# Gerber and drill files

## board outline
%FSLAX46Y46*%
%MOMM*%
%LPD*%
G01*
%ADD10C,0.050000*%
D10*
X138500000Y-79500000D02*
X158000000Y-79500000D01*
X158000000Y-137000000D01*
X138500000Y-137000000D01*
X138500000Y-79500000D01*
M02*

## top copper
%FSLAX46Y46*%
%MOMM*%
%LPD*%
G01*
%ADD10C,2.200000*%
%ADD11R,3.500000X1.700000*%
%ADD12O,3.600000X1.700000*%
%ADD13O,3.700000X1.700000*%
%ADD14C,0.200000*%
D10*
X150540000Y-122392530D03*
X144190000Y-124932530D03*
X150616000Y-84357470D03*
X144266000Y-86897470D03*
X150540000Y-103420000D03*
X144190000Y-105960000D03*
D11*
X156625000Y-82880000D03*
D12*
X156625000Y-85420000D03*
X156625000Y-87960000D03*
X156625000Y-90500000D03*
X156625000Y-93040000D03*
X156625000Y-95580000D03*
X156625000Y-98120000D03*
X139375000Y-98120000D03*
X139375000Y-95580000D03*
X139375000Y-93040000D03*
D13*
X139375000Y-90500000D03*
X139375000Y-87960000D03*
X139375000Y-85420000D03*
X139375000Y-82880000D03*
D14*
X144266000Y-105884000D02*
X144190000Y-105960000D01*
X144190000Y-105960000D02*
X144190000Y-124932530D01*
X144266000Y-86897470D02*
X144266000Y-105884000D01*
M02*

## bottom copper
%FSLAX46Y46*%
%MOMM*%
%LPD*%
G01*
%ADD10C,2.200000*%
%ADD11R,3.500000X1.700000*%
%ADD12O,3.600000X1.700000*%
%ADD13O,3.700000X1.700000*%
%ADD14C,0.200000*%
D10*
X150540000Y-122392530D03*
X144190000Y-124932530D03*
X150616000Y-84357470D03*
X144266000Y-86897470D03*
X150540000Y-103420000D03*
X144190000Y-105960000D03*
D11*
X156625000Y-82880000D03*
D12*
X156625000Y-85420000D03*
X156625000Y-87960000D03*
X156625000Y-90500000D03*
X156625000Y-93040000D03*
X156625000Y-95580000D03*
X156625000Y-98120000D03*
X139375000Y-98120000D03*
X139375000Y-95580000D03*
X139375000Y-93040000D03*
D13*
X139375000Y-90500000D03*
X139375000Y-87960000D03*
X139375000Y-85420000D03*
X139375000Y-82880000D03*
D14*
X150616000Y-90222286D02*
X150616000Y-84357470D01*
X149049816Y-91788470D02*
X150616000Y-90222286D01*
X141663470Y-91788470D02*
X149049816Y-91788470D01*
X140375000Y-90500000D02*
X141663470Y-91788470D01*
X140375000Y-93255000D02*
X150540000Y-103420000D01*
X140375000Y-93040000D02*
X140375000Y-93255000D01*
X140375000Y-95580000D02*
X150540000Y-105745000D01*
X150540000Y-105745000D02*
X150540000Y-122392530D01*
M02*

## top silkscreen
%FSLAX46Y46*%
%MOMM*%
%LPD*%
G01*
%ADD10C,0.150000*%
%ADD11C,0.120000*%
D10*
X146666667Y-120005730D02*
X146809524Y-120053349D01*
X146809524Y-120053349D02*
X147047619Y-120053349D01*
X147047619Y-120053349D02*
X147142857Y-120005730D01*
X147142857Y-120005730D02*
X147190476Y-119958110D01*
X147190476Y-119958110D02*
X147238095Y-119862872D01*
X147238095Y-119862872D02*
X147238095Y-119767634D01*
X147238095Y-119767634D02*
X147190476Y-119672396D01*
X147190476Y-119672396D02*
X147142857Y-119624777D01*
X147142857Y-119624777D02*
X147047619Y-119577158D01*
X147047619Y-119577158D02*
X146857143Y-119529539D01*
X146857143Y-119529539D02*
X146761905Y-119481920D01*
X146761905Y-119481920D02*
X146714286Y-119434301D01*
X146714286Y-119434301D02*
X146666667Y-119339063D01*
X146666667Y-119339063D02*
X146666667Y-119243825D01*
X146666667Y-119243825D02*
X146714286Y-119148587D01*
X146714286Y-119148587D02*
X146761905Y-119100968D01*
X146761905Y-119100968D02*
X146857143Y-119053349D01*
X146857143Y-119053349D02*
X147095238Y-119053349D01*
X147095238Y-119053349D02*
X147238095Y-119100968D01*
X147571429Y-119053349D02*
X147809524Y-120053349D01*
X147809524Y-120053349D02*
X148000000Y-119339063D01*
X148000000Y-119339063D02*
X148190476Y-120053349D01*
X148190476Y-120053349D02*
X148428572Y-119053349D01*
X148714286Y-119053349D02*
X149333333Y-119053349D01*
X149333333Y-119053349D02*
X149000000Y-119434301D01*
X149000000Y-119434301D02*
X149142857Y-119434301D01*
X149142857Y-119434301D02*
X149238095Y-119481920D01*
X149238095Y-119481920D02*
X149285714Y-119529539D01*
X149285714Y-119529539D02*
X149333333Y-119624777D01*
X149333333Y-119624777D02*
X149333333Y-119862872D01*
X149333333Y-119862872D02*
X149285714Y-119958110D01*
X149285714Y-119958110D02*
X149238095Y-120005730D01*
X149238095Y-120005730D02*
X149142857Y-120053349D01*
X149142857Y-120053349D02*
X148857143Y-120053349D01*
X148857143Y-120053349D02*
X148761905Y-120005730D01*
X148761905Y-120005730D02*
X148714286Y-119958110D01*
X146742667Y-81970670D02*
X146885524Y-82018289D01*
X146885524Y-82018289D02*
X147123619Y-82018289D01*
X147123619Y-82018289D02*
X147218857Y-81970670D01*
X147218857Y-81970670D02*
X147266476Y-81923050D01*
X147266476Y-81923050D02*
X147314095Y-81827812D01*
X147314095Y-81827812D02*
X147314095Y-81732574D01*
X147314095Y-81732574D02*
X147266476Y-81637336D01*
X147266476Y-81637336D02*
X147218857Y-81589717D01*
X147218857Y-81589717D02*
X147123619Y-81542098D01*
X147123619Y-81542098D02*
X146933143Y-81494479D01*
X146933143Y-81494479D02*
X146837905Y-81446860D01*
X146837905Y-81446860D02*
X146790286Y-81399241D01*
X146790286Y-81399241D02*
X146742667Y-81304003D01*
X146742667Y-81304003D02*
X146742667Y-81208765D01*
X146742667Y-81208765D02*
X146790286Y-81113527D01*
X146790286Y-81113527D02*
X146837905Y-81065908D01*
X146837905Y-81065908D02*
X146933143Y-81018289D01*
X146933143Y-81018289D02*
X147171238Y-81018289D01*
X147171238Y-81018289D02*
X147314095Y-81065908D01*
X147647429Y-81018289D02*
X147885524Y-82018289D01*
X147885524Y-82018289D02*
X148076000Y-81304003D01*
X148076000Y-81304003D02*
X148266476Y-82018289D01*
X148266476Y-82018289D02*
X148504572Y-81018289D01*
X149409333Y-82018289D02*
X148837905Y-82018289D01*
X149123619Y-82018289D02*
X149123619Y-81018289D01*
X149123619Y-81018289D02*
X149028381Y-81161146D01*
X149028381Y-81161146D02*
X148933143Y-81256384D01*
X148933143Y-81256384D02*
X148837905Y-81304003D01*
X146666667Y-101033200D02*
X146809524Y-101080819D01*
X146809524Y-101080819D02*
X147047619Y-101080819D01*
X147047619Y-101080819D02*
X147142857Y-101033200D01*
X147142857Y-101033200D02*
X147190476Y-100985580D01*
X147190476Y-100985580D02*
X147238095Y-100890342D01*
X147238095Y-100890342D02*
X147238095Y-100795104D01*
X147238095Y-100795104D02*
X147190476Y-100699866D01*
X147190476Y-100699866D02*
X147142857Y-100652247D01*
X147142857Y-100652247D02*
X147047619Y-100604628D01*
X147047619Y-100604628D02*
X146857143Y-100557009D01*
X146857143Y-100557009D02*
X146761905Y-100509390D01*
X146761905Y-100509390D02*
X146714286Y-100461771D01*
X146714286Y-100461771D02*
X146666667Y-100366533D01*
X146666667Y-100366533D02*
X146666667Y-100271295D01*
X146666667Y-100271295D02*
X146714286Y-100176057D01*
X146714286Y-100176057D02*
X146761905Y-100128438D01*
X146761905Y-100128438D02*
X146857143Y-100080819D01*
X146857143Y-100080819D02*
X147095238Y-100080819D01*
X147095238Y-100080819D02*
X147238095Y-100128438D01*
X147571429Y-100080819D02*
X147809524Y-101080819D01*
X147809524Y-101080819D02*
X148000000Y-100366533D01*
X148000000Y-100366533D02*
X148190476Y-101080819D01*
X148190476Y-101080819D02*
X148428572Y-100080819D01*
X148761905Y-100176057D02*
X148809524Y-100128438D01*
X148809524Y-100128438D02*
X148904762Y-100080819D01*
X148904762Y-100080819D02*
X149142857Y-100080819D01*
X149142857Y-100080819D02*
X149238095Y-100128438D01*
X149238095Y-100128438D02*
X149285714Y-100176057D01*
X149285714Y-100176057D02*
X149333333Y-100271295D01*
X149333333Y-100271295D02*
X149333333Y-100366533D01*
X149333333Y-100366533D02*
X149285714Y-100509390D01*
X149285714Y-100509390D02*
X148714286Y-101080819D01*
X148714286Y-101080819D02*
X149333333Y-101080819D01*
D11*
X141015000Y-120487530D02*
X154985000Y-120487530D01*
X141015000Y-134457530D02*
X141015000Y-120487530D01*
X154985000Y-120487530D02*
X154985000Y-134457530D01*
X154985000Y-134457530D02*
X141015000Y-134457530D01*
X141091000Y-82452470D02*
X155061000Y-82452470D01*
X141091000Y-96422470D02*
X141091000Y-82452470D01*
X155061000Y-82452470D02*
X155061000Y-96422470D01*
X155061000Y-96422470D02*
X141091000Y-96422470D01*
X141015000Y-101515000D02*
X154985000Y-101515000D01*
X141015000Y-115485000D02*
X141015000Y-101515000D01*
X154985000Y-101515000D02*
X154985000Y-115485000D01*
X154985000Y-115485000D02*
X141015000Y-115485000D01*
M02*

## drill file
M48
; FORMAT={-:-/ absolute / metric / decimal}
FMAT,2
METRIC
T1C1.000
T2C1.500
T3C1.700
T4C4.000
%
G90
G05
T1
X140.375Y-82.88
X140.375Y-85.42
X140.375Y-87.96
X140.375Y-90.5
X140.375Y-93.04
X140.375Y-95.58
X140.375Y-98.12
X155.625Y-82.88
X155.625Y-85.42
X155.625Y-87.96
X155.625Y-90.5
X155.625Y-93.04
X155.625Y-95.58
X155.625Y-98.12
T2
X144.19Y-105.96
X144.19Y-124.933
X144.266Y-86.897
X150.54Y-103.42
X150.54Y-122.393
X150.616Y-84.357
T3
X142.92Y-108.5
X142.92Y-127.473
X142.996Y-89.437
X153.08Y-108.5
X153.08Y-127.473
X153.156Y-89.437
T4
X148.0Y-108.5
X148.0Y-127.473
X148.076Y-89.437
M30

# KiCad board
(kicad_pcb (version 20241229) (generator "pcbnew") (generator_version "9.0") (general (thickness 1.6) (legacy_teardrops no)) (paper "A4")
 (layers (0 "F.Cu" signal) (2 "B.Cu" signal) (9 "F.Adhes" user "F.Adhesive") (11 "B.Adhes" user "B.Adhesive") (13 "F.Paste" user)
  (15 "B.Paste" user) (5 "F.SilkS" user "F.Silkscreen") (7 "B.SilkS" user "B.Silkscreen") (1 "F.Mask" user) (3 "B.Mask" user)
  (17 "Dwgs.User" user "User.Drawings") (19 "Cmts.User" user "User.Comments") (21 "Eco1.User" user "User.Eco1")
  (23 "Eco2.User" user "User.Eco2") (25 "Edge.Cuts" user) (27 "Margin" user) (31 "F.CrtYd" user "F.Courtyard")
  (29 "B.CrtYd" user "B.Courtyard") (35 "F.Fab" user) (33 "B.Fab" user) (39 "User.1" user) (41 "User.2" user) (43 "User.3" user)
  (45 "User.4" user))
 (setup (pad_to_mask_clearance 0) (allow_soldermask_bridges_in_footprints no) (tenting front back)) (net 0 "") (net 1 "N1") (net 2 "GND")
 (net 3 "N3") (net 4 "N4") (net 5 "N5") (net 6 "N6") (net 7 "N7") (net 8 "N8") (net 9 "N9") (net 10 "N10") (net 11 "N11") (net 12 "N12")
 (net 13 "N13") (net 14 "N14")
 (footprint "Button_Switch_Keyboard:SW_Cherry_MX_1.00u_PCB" (layer "F.Cu") (at 150.54 122.39253)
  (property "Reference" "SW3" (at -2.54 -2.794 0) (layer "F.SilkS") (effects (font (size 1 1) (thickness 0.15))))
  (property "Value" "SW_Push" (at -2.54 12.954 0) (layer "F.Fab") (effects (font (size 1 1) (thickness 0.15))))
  (fp_line (start -9.525 -1.905) (end 4.445 -1.905) (stroke (width 0.12) (type solid)) (layer "F.SilkS"))
  (fp_line (start -9.525 12.065) (end -9.525 -1.905) (stroke (width 0.12) (type solid)) (layer "F.SilkS"))
  (fp_line (start 4.445 -1.905) (end 4.445 12.065) (stroke (width 0.12) (type solid)) (layer "F.SilkS"))
  (fp_line (start 4.445 12.065) (end -9.525 12.065) (stroke (width 0.12) (type solid)) (layer "F.SilkS"))
  (pad "" np_thru_hole circle (at -7.62 5.08) (size 1.7 1.7) (drill 1.7) (layers "*.Cu" "*.Mask"))
  (pad "" np_thru_hole circle (at -2.54 5.08) (size 4 4) (drill 4) (layers "*.Cu" "*.Mask"))
  (pad "" np_thru_hole circle (at 2.54 5.08) (size 1.7 1.7) (drill 1.7) (layers "*.Cu" "*.Mask"))
  (pad "1" thru_hole circle (at 0 0) (size 2.2 2.2) (drill 1.5) (layers "*.Cu" "*.Mask") (remove_unused_layers no) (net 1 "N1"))
  (pad "2" thru_hole circle (at -6.35 2.54) (size 2.2 2.2) (drill 1.5) (layers "*.Cu" "*.Mask") (remove_unused_layers no) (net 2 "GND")))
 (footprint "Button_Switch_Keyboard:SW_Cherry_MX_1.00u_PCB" (layer "F.Cu") (at 150.616 84.35747)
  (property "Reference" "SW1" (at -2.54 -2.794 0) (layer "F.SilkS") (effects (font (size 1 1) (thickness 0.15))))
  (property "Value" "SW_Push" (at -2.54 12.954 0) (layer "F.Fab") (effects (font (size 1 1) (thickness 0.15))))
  (fp_line (start -9.525 -1.905) (end 4.445 -1.905) (stroke (width 0.12) (type solid)) (layer "F.SilkS"))
  (fp_line (start -9.525 12.065) (end -9.525 -1.905) (stroke (width 0.12) (type solid)) (layer "F.SilkS"))
  (fp_line (start 4.445 -1.905) (end 4.445 12.065) (stroke (width 0.12) (type solid)) (layer "F.SilkS"))
  (fp_line (start 4.445 12.065) (end -9.525 12.065) (stroke (width 0.12) (type solid)) (layer "F.SilkS"))
  (pad "" np_thru_hole circle (at -7.62 5.08) (size 1.7 1.7) (drill 1.7) (layers "*.Cu" "*.Mask"))
  (pad "" np_thru_hole circle (at -2.54 5.08) (size 4 4) (drill 4) (layers "*.Cu" "*.Mask"))
  (pad "" np_thru_hole circle (at 2.54 5.08) (size 1.7 1.7) (drill 1.7) (layers "*.Cu" "*.Mask"))
  (pad "1" thru_hole circle (at 0 0) (size 2.2 2.2) (drill 1.5) (layers "*.Cu" "*.Mask") (remove_unused_layers no) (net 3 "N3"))
  (pad "2" thru_hole circle (at -6.35 2.54) (size 2.2 2.2) (drill 1.5) (layers "*.Cu" "*.Mask") (remove_unused_layers no) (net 2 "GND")))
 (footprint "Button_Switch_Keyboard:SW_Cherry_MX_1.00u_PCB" (layer "F.Cu") (at 150.54 103.42)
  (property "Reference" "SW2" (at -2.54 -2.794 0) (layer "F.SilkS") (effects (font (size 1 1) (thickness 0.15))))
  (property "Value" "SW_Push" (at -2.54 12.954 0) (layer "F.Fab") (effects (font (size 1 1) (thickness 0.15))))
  (fp_line (start -9.525 -1.905) (end 4.445 -1.905) (stroke (width 0.12) (type solid)) (layer "F.SilkS"))
  (fp_line (start -9.525 12.065) (end -9.525 -1.905) (stroke (width 0.12) (type solid)) (layer "F.SilkS"))
  (fp_line (start 4.445 -1.905) (end 4.445 12.065) (stroke (width 0.12) (type solid)) (layer "F.SilkS"))
  (fp_line (start 4.445 12.065) (end -9.525 12.065) (stroke (width 0.12) (type solid)) (layer "F.SilkS"))
  (pad "" np_thru_hole circle (at -7.62 5.08) (size 1.7 1.7) (drill 1.7) (layers "*.Cu" "*.Mask"))
  (pad "" np_thru_hole circle (at -2.54 5.08) (size 4 4) (drill 4) (layers "*.Cu" "*.Mask"))
  (pad "" np_thru_hole circle (at 2.54 5.08) (size 1.7 1.7) (drill 1.7) (layers "*.Cu" "*.Mask"))
  (pad "1" thru_hole circle (at 0 0) (size 2.2 2.2) (drill 1.5) (layers "*.Cu" "*.Mask") (remove_unused_layers no) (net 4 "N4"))
  (pad "2" thru_hole circle (at -6.35 2.54) (size 2.2 2.2) (drill 1.5) (layers "*.Cu" "*.Mask") (remove_unused_layers no) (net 2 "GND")))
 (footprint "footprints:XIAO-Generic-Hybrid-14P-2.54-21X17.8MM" (layer "B.Cu") (at 148 90.5 180)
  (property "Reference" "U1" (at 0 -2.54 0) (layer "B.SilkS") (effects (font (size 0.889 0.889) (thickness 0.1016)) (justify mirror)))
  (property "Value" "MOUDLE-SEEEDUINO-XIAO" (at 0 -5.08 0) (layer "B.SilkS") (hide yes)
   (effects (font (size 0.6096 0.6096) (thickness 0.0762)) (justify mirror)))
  (pad "1" thru_hole rect (at -7.625 7.62 180) (size 3.5 1.7) (drill 1 (offset -1 0)) (layers "*.Cu" "*.Mask") (remove_unused_layers no)
   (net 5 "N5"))
  (pad "2" thru_hole oval (at -7.625 5.08 180) (size 3.6 1.7) (drill 1 (offset -1 0)) (layers "*.Cu" "*.Mask") (remove_unused_layers no)
   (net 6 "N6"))
  (pad "3" thru_hole oval (at -7.625 2.54 180) (size 3.6 1.7) (drill 1 (offset -1 0)) (layers "*.Cu" "*.Mask") (remove_unused_layers no)
   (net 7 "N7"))
  (pad "4" thru_hole oval (at -7.625 0 180) (size 3.6 1.7) (drill 1 (offset -1 0)) (layers "*.Cu" "*.Mask") (remove_unused_layers no)
   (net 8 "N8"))
  (pad "5" thru_hole oval (at -7.625 -2.54 180) (size 3.6 1.7) (drill 1 (offset -1 0)) (layers "*.Cu" "*.Mask") (remove_unused_layers no)
   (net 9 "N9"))
  (pad "6" thru_hole oval (at -7.625 -5.08) (size 3.6 1.7) (drill 1 (offset 1 0)) (layers "*.Cu" "*.Mask") (remove_unused_layers no)
   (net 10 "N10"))
  (pad "7" thru_hole oval (at -7.625 -7.62 180) (size 3.6 1.7) (drill 1 (offset -1 0)) (layers "*.Cu" "*.Mask") (remove_unused_layers no)
   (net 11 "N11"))
  (pad "8" thru_hole oval (at 7.625 -7.62 180) (size 3.6 1.7) (drill 1 (offset 1 0)) (layers "*.Cu" "*.Mask") (remove_unused_layers no)
   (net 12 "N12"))
  (pad "9" thru_hole oval (at 7.625 -5.08 180) (size 3.6 1.7) (drill 1 (offset 1 0)) (layers "*.Cu" "*.Mask") (remove_unused_layers no)
   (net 1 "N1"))
  (pad "10" thru_hole oval (at 7.625 -2.54 180) (size 3.6 1.7) (drill 1 (offset 1 0)) (layers "*.Cu" "*.Mask") (remove_unused_layers no)
   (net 4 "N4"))
  (pad "11" thru_hole oval (at 7.625 0 180) (size 3.7 1.7) (drill 1 (offset 1 0)) (layers "*.Cu" "*.Mask") (remove_unused_layers no)
   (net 3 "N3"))
  (pad "12" thru_hole oval (at 7.625 2.54 180) (size 3.7 1.7) (drill 1 (offset 1 0)) (layers "*.Cu" "*.Mask") (remove_unused_layers no)
   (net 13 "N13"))
  (pad "13" thru_hole oval (at 7.625 5.08 180) (size 3.7 1.7) (drill 1 (offset 1 0)) (layers "*.Cu" "*.Mask") (remove_unused_layers no)
   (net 2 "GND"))
  (pad "14" thru_hole oval (at 7.625 7.62 180) (size 3.7 1.7) (drill 1 (offset 1 0)) (layers "*.Cu" "*.Mask") (remove_unused_layers no)
   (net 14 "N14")))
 (gr_rect (start 138.5 79.5) (end 158 137) (stroke (width 0.05) (type default)) (fill no) (layer "Edge.Cuts"))
 (segment (start 144.266 105.884) (end 144.19 105.96) (width 0.2) (layer "F.Cu") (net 2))
 (segment (start 144.19 105.96) (end 144.19 124.93253) (width 0.2) (layer "F.Cu") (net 2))
 (segment (start 144.266 86.89747) (end 144.266 105.884) (width 0.2) (layer "F.Cu") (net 2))
 (segment (start 150.616 90.222286) (end 150.616 84.35747) (width 0.2) (layer "B.Cu") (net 3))
 (segment (start 149.049816 91.78847) (end 150.616 90.222286) (width 0.2) (layer "B.Cu") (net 3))
 (segment (start 141.66347 91.78847) (end 149.049816 91.78847) (width 0.2) (layer "B.Cu") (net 3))
 (segment (start 140.375 90.5) (end 141.66347 91.78847) (width 0.2) (layer "B.Cu") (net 3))
 (segment (start 140.375 93.255) (end 150.54 103.42) (width 0.2) (layer "B.Cu") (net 4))
 (segment (start 140.375 93.04) (end 140.375 93.255) (width 0.2) (layer "B.Cu") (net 4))
 (segment (start 140.375 95.58) (end 150.54 105.745) (width 0.2) (layer "B.Cu") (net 1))
 (segment (start 150.54 105.745) (end 150.54 122.39253) (width 0.2) (layer "B.Cu") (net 1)))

